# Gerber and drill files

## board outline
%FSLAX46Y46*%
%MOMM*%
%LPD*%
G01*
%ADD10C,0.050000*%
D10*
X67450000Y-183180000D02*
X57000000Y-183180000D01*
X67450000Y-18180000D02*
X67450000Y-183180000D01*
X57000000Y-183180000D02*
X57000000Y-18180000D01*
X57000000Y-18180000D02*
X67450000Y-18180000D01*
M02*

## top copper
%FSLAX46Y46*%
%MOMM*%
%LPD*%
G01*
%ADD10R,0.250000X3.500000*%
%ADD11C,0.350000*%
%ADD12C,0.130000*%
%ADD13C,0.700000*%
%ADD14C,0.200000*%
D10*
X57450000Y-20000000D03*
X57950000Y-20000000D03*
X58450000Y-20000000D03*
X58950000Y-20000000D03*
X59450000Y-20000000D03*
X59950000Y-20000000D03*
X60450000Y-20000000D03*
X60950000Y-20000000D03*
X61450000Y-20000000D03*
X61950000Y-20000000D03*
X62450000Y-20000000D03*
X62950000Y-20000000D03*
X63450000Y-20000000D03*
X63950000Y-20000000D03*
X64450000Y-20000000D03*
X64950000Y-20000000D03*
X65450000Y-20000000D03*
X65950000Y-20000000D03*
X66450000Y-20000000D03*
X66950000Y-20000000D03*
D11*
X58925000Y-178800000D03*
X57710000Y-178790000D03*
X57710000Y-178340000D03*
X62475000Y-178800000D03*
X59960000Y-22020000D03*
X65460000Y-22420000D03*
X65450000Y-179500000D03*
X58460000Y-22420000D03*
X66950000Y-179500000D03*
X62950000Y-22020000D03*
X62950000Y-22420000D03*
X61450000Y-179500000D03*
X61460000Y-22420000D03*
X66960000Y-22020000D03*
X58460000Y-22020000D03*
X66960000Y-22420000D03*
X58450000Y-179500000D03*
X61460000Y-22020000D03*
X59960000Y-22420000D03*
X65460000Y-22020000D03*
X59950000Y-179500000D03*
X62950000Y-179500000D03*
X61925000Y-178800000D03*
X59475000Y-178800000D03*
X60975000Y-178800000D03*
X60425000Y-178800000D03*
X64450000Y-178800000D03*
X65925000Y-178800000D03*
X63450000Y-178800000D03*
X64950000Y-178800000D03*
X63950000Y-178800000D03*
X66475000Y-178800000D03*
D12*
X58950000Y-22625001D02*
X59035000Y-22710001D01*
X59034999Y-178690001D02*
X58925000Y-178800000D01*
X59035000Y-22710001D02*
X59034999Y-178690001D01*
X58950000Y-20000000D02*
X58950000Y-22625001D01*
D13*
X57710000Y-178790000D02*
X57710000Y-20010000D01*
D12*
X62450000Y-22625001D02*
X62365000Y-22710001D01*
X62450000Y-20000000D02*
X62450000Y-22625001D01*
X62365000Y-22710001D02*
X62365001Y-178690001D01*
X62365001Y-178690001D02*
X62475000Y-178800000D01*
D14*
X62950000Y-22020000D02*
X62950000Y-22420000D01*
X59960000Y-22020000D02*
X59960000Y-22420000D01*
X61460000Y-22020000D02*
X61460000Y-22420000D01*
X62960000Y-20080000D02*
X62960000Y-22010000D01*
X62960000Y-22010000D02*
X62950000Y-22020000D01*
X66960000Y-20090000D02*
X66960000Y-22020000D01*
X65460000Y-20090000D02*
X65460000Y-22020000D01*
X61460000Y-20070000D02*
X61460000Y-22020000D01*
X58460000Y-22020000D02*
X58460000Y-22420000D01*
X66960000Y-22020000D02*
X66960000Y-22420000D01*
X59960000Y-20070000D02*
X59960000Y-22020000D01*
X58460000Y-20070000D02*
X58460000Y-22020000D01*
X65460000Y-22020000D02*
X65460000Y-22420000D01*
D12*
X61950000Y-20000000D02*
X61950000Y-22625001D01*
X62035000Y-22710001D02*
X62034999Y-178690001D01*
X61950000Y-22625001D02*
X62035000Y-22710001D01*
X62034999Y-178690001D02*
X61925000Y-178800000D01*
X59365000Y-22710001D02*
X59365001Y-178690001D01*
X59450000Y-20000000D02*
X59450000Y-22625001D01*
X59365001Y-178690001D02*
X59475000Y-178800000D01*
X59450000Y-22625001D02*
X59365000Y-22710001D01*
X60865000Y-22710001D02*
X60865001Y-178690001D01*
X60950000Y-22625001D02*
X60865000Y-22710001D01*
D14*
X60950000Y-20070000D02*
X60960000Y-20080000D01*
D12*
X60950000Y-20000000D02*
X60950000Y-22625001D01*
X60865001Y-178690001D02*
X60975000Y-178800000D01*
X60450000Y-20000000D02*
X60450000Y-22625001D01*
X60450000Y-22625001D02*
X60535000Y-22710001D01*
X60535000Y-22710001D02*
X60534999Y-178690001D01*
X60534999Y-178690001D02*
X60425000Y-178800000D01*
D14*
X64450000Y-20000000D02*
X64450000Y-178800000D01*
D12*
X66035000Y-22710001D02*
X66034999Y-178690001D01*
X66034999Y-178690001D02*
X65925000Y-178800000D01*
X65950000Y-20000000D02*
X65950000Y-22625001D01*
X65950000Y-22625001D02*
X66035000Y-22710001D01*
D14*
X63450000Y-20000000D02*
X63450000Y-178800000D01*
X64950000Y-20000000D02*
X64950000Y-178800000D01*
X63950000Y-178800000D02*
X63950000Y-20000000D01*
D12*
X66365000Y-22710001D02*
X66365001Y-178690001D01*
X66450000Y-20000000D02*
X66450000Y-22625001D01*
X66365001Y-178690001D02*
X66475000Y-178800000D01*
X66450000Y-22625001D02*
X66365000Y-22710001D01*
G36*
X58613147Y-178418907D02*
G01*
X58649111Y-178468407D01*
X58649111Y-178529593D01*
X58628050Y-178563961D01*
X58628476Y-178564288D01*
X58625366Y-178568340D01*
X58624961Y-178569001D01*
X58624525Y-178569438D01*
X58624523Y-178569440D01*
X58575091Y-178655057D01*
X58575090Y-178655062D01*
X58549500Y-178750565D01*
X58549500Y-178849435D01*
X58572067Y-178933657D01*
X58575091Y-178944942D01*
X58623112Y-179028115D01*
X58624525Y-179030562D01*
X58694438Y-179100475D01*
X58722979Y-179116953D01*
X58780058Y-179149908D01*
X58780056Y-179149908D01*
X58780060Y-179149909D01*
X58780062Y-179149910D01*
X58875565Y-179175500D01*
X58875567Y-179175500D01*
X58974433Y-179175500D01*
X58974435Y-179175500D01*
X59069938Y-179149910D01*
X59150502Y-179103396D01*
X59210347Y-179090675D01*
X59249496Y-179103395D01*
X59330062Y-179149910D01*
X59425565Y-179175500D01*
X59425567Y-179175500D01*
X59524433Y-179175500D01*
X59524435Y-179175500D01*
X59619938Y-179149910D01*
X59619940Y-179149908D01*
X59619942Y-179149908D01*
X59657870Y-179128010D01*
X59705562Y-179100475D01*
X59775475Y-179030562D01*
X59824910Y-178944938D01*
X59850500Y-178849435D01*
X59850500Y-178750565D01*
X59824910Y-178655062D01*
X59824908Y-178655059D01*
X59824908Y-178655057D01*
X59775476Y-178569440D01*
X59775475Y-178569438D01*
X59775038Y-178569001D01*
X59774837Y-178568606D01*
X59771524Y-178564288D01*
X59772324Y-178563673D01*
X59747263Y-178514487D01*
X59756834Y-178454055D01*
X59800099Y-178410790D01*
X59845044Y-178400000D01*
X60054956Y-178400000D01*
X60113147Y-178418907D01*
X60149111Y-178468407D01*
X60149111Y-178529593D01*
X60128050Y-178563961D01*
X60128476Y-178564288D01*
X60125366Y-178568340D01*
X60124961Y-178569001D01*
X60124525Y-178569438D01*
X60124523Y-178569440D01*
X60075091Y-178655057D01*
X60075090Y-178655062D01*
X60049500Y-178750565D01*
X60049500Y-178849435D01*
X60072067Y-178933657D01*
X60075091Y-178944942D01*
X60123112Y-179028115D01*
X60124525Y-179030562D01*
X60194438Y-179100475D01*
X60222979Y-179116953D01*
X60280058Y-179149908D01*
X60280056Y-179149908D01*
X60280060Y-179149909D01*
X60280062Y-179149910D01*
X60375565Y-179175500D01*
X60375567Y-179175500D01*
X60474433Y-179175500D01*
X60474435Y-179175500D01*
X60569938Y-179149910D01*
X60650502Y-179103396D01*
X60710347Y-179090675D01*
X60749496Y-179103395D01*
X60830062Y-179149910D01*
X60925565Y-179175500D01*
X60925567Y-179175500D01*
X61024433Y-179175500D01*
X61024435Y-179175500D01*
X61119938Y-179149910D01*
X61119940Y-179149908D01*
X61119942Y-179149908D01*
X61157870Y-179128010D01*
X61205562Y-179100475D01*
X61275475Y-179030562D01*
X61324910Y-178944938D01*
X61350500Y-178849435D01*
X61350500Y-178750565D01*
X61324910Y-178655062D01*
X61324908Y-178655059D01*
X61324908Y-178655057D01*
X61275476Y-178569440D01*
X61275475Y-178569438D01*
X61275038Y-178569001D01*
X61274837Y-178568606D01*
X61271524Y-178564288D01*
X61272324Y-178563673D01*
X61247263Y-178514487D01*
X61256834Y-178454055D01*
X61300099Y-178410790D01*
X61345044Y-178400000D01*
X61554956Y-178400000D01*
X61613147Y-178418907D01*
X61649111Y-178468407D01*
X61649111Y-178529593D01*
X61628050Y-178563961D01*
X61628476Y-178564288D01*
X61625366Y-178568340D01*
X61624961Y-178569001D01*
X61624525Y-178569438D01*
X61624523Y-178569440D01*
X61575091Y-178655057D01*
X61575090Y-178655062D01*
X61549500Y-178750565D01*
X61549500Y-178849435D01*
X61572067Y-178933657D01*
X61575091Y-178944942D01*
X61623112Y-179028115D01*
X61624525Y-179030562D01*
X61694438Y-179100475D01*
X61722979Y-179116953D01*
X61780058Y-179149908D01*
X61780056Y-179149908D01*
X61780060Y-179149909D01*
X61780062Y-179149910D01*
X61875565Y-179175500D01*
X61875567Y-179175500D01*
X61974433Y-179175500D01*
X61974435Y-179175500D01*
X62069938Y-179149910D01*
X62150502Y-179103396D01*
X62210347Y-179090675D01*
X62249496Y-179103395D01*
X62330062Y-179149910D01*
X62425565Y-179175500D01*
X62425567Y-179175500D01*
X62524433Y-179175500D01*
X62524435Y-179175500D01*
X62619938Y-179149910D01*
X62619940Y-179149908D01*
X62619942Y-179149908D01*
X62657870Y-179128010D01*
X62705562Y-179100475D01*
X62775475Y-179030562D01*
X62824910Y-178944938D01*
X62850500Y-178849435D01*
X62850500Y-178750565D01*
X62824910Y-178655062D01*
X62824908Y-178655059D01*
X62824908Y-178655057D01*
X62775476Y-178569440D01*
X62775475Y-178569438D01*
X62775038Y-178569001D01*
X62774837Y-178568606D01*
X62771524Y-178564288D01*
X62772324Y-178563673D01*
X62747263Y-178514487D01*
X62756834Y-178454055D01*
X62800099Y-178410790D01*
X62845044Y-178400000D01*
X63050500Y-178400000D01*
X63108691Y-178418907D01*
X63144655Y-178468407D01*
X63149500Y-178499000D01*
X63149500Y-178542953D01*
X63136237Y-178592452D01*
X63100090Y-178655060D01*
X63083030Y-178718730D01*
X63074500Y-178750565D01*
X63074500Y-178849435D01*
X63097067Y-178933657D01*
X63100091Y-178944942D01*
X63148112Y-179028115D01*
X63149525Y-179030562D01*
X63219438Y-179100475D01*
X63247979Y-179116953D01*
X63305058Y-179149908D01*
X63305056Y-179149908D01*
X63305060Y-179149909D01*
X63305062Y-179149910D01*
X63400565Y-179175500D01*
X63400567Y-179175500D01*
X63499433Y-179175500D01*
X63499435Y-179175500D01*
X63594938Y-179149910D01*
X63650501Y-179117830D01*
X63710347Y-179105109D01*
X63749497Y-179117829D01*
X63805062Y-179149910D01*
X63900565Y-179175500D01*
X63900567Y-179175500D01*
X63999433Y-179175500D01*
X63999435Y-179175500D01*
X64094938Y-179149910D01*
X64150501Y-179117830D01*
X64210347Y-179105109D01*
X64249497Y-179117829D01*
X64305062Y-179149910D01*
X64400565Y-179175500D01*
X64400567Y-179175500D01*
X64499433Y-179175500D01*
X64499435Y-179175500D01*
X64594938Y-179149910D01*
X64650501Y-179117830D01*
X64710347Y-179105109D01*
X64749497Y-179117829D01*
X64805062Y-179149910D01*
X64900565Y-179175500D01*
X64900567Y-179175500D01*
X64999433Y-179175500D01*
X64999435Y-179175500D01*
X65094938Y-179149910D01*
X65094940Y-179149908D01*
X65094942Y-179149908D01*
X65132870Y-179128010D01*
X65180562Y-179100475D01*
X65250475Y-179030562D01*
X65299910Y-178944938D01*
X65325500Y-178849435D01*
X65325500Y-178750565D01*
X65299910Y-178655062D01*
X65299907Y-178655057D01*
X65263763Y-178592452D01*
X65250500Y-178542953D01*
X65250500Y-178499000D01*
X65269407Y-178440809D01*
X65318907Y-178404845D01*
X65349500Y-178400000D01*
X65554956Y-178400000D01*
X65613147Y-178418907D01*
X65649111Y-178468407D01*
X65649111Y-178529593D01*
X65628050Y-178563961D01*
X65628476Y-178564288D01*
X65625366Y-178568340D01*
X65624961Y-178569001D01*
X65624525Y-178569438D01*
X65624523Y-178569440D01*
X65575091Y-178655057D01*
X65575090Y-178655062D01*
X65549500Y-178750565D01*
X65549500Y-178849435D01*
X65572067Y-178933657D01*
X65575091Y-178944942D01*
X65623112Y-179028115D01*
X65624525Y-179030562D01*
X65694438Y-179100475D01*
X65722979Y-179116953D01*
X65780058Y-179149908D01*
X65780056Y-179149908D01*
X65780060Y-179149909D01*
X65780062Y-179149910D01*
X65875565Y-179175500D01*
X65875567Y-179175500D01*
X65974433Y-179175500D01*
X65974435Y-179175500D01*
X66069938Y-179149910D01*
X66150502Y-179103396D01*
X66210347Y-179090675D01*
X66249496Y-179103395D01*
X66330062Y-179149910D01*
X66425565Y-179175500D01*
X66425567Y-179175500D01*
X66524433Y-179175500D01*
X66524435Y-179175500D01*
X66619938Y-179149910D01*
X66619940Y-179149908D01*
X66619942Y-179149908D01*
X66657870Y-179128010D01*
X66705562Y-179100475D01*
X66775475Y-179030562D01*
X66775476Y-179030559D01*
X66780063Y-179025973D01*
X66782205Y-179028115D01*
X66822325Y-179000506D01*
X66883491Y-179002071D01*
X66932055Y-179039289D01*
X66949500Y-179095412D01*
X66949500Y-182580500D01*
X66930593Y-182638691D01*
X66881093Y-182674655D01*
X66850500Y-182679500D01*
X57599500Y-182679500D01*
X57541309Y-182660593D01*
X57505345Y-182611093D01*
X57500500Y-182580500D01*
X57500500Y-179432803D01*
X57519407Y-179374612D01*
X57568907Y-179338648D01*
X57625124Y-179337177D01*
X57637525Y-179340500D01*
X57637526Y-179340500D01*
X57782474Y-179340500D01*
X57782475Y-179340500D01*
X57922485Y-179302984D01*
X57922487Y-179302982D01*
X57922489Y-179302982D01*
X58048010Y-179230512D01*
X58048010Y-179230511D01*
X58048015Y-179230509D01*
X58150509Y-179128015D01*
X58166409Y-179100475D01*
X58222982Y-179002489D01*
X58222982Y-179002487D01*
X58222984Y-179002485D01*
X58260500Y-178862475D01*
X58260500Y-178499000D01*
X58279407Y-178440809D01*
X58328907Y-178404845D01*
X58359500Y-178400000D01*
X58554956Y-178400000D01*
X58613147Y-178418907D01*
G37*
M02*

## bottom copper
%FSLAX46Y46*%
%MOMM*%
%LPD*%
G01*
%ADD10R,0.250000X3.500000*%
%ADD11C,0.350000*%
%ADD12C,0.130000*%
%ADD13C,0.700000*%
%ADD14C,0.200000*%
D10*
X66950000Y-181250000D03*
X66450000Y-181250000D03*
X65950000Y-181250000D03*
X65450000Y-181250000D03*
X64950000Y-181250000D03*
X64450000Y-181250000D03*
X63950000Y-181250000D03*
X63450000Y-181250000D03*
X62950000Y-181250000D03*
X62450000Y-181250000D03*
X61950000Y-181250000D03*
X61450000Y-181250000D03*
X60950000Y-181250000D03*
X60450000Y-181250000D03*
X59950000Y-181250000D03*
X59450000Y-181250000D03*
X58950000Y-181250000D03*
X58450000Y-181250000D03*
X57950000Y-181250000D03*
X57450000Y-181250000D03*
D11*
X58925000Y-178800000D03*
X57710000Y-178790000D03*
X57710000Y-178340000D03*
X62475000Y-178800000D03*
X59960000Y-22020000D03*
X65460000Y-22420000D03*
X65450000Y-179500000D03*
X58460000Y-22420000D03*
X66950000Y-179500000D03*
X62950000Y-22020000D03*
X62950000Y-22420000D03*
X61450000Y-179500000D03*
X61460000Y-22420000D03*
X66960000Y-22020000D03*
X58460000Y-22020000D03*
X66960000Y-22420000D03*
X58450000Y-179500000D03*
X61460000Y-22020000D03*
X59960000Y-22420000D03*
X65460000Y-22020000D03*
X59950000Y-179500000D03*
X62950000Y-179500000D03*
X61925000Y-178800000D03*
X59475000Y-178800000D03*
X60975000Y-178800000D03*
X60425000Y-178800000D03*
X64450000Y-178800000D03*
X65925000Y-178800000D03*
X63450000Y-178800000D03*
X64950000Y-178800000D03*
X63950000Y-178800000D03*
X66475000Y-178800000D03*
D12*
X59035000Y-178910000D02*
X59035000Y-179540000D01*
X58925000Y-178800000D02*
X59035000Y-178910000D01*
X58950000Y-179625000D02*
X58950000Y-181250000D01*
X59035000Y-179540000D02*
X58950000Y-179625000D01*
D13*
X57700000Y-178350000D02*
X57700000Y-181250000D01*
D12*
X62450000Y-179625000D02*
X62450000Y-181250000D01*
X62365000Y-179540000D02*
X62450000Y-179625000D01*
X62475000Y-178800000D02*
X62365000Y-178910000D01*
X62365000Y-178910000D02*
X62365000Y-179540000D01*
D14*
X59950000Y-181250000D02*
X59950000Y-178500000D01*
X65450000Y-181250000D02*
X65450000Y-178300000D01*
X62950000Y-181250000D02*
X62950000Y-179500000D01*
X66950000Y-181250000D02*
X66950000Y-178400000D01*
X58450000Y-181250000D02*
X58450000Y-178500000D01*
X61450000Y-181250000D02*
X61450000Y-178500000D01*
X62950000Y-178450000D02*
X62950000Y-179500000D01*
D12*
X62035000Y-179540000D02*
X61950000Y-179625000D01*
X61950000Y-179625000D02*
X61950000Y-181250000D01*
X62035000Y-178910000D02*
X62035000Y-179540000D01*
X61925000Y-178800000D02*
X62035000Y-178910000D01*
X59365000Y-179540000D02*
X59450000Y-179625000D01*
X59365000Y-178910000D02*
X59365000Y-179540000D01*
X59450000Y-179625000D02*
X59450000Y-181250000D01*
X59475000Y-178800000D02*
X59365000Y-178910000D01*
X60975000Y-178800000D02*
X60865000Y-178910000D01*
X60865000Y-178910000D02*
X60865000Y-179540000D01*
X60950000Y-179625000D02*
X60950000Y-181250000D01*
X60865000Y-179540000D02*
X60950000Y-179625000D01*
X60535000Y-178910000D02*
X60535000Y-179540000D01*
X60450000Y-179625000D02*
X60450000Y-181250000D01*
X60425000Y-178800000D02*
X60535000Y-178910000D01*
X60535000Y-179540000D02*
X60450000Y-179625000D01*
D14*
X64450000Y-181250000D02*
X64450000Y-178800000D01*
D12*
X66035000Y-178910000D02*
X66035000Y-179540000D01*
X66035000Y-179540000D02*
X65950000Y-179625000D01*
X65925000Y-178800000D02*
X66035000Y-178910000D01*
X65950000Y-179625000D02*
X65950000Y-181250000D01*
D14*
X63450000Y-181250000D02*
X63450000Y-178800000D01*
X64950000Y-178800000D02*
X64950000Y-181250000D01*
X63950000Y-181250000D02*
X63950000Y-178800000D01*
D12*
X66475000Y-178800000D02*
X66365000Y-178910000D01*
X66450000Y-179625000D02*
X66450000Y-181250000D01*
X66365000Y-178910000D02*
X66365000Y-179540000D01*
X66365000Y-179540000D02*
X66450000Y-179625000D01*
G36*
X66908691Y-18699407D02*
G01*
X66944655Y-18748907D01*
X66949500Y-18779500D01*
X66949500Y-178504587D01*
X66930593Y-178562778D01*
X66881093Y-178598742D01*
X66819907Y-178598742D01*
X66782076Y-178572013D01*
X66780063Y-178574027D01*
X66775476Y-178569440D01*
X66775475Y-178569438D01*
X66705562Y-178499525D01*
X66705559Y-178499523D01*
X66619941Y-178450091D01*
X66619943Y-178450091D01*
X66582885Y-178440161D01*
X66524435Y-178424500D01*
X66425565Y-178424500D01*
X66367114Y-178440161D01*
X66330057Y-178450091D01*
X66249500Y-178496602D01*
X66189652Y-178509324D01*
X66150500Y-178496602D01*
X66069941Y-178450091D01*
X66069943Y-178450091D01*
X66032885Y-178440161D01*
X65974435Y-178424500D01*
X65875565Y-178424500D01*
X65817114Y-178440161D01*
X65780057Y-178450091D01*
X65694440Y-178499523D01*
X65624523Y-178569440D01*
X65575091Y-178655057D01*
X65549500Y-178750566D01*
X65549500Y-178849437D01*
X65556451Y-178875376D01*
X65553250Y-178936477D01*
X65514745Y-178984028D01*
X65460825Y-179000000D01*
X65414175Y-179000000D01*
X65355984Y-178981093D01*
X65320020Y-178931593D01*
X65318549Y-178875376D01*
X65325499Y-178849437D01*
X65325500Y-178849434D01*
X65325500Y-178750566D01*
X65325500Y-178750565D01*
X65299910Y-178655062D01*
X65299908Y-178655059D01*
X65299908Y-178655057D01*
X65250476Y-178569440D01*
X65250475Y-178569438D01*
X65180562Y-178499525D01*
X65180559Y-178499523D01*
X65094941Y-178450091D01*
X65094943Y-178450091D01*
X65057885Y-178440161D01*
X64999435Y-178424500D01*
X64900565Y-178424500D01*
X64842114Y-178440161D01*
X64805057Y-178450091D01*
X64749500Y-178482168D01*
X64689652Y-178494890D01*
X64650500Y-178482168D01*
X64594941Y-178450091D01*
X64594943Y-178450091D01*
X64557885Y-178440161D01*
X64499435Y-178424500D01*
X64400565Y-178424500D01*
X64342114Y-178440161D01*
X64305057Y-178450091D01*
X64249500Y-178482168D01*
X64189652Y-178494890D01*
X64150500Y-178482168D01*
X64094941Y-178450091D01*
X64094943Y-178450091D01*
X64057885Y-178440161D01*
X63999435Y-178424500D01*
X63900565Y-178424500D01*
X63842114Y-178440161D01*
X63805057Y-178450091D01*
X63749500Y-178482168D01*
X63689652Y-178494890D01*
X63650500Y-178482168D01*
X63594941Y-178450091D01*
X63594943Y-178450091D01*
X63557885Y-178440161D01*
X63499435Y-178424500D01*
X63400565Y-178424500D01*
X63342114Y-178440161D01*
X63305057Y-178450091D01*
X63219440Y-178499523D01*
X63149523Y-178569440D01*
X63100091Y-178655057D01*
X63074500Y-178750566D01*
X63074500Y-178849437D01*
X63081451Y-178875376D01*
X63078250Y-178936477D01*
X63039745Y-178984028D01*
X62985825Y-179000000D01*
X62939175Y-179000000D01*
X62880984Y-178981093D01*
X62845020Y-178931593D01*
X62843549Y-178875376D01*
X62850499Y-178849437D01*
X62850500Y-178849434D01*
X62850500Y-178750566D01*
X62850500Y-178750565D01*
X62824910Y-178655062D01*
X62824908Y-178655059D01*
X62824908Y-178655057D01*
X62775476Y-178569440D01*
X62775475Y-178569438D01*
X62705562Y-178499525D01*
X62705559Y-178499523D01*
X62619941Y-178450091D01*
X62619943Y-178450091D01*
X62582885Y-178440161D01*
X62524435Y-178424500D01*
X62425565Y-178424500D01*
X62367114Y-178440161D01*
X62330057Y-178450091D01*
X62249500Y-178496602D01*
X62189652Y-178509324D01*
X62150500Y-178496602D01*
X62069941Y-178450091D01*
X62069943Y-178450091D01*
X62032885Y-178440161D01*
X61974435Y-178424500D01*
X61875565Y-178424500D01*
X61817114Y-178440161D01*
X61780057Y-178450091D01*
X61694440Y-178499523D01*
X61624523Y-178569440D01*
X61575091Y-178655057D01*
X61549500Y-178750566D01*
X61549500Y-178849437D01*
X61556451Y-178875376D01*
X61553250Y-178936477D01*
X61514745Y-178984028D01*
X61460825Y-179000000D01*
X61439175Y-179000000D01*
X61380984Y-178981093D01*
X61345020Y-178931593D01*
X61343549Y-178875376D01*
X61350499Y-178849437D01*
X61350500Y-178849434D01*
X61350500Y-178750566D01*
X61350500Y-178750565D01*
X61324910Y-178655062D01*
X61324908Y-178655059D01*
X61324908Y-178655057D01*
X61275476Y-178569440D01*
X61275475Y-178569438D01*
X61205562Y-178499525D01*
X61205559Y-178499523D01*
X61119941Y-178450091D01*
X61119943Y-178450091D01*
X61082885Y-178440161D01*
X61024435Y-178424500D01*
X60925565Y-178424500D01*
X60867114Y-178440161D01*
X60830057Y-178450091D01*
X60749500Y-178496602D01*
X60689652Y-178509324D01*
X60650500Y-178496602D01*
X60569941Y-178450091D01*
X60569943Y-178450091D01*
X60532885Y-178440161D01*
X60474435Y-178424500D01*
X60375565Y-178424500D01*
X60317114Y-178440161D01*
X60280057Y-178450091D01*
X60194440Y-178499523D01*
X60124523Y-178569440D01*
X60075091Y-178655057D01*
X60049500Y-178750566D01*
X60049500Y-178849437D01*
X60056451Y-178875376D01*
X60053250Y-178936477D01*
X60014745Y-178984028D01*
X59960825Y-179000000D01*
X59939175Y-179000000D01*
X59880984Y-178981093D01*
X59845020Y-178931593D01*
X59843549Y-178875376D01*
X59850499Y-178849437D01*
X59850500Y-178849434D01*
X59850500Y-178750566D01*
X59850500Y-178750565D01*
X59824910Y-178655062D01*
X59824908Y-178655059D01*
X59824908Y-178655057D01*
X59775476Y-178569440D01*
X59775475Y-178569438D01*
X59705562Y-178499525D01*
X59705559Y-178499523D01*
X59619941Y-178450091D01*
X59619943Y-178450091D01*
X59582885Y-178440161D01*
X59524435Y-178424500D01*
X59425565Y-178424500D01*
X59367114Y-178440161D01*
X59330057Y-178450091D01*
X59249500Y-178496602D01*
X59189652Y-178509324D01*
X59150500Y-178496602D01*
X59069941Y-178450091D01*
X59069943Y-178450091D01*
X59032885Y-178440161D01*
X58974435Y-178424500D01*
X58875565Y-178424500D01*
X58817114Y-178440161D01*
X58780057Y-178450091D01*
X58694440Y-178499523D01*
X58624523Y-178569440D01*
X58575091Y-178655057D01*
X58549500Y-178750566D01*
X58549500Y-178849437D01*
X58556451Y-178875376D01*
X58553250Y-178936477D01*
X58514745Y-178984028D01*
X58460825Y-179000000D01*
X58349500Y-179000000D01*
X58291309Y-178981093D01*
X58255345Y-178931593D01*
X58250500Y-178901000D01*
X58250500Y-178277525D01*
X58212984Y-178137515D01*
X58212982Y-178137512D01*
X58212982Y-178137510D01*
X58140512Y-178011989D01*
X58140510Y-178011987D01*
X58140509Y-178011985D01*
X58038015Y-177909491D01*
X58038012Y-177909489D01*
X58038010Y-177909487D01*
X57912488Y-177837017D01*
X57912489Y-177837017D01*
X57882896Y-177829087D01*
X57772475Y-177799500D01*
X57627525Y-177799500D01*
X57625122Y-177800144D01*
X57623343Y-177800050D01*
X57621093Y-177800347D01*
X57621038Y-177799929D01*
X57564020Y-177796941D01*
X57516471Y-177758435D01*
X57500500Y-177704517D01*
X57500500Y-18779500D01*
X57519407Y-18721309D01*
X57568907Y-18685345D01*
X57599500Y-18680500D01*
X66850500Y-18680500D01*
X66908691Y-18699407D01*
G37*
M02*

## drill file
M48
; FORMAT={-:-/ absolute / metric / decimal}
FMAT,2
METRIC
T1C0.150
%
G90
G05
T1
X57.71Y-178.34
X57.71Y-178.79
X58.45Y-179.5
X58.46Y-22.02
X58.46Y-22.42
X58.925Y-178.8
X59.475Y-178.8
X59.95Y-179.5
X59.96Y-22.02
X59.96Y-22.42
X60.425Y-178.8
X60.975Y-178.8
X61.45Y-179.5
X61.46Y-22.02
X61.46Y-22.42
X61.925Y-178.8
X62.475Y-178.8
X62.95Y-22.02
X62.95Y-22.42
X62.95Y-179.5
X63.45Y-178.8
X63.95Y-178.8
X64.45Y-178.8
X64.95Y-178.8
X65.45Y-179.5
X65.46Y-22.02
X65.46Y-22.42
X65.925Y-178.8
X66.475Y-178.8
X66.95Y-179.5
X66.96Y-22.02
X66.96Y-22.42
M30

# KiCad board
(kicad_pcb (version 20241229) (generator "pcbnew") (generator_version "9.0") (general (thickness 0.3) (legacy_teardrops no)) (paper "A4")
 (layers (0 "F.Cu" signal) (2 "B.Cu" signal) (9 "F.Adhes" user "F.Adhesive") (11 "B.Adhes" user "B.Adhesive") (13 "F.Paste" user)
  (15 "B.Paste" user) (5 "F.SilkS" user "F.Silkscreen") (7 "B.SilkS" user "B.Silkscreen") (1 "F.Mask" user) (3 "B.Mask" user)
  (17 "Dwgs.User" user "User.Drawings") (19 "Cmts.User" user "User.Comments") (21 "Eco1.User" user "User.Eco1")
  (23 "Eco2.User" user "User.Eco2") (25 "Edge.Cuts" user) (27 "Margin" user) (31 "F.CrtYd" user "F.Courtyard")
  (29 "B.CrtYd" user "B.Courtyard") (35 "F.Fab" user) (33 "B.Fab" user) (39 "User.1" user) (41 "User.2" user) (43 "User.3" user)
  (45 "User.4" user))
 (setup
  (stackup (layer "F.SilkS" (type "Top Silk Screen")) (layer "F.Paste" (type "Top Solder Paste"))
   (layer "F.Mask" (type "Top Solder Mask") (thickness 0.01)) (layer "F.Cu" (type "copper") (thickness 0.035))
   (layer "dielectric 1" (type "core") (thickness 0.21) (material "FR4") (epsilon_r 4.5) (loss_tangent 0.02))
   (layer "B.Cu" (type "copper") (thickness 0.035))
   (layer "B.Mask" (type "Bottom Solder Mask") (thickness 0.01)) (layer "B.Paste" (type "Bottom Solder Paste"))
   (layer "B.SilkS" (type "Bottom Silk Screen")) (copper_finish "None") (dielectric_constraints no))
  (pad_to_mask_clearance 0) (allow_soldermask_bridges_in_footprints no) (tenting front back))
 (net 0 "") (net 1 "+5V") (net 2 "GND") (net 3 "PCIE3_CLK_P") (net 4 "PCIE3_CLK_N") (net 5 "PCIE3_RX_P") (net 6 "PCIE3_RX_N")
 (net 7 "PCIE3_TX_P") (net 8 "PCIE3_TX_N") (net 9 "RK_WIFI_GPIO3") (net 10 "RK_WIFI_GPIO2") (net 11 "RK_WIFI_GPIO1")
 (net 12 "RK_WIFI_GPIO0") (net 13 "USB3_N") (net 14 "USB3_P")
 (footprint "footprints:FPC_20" (layer "F.Cu") (at 62.2 20 180)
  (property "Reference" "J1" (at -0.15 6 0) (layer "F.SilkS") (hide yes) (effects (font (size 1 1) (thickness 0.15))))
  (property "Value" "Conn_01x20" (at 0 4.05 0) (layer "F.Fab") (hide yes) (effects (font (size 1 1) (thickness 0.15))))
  (pad "1" smd rect (at 4.75 0 180) (size 0.25 3.5) (layers "F.Cu" "F.Mask" "F.Paste") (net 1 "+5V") (thermal_bridge_angle 45))
  (pad "2" smd rect (at 4.25 0 180) (size 0.25 3.5) (layers "F.Cu" "F.Mask" "F.Paste") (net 1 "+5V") (thermal_bridge_angle 45))
  (pad "3" smd rect (at 3.75 0 180) (size 0.25 3.5) (layers "F.Cu" "F.Mask" "F.Paste") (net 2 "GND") (thermal_bridge_angle 45))
  (pad "4" smd rect (at 3.25 0 180) (size 0.25 3.5) (layers "F.Cu" "F.Mask" "F.Paste") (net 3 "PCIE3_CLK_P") (thermal_bridge_angle 45))
  (pad "5" smd rect (at 2.75 0 180) (size 0.25 3.5) (layers "F.Cu" "F.Mask" "F.Paste") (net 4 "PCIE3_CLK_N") (thermal_bridge_angle 45))
  (pad "6" smd rect (at 2.25 0 180) (size 0.25 3.5) (layers "F.Cu" "F.Mask" "F.Paste") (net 2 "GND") (thermal_bridge_angle 45))
  (pad "7" smd rect (at 1.75 0 180) (size 0.25 3.5) (layers "F.Cu" "F.Mask" "F.Paste") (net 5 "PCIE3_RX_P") (thermal_bridge_angle 45))
  (pad "8" smd rect (at 1.25 0 180) (size 0.25 3.5) (layers "F.Cu" "F.Mask" "F.Paste") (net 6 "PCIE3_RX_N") (thermal_bridge_angle 45))
  (pad "9" smd rect (at 0.75 0 180) (size 0.25 3.5) (layers "F.Cu" "F.Mask" "F.Paste") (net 2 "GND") (thermal_bridge_angle 45))
  (pad "10" smd rect (at 0.25 0 180) (size 0.25 3.5) (layers "F.Cu" "F.Mask" "F.Paste") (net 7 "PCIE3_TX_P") (thermal_bridge_angle 45))
  (pad "11" smd rect (at -0.25 0 180) (size 0.25 3.5) (layers "F.Cu" "F.Mask" "F.Paste") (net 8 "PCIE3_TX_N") (thermal_bridge_angle 45))
  (pad "12" smd rect (at -0.75 0 180) (size 0.25 3.5) (layers "F.Cu" "F.Mask" "F.Paste") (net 2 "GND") (thermal_bridge_angle 45))
  (pad "13" smd rect (at -1.25 0 180) (size 0.25 3.5) (layers "F.Cu" "F.Mask" "F.Paste") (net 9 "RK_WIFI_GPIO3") (thermal_bridge_angle 45))
  (pad "14" smd rect (at -1.75 0 180) (size 0.25 3.5) (layers "F.Cu" "F.Mask" "F.Paste") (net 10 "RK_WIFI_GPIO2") (thermal_bridge_angle 45))
  (pad "15" smd rect (at -2.25 0 180) (size 0.25 3.5) (layers "F.Cu" "F.Mask" "F.Paste") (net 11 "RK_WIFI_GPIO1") (thermal_bridge_angle 45))
  (pad "16" smd rect (at -2.75 0 180) (size 0.25 3.5) (layers "F.Cu" "F.Mask" "F.Paste") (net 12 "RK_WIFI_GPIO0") (thermal_bridge_angle 45))
  (pad "17" smd rect (at -3.25 0 180) (size 0.25 3.5) (layers "F.Cu" "F.Mask" "F.Paste") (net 2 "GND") (thermal_bridge_angle 45))
  (pad "18" smd rect (at -3.75 0 180) (size 0.25 3.5) (layers "F.Cu" "F.Mask" "F.Paste") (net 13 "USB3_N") (thermal_bridge_angle 45))
  (pad "19" smd rect (at -4.25 0 180) (size 0.25 3.5) (layers "F.Cu" "F.Mask" "F.Paste") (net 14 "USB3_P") (thermal_bridge_angle 45))
  (pad "20" smd rect (at -4.75 0 180) (size 0.25 3.5) (layers "F.Cu" "F.Mask" "F.Paste") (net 2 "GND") (thermal_bridge_angle 45)))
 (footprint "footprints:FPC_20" (layer "B.Cu") (at 62.2 181.25)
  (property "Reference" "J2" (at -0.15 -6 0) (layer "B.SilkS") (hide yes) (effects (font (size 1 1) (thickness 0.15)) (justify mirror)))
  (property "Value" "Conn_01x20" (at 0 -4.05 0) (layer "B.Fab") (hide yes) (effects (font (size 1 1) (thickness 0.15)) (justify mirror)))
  (pad "1" smd rect (at 4.75 0) (size 0.25 3.5) (layers "B.Cu" "B.Mask" "B.Paste") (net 2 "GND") (thermal_bridge_angle 45))
  (pad "2" smd rect (at 4.25 0) (size 0.25 3.5) (layers "B.Cu" "B.Mask" "B.Paste") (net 14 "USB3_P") (thermal_bridge_angle 45))
  (pad "3" smd rect (at 3.75 0) (size 0.25 3.5) (layers "B.Cu" "B.Mask" "B.Paste") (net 13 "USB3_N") (thermal_bridge_angle 45))
  (pad "4" smd rect (at 3.25 0) (size 0.25 3.5) (layers "B.Cu" "B.Mask" "B.Paste") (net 2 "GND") (thermal_bridge_angle 45))
  (pad "5" smd rect (at 2.75 0) (size 0.25 3.5) (layers "B.Cu" "B.Mask" "B.Paste") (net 12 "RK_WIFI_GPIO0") (thermal_bridge_angle 45))
  (pad "6" smd rect (at 2.25 0) (size 0.25 3.5) (layers "B.Cu" "B.Mask" "B.Paste") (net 11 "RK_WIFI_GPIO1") (thermal_bridge_angle 45))
  (pad "7" smd rect (at 1.75 0) (size 0.25 3.5) (layers "B.Cu" "B.Mask" "B.Paste") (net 10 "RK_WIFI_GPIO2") (thermal_bridge_angle 45))
  (pad "8" smd rect (at 1.25 0) (size 0.25 3.5) (layers "B.Cu" "B.Mask" "B.Paste") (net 9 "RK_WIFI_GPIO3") (thermal_bridge_angle 45))
  (pad "9" smd rect (at 0.75 0) (size 0.25 3.5) (layers "B.Cu" "B.Mask" "B.Paste") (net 2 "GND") (thermal_bridge_angle 45))
  (pad "10" smd rect (at 0.25 0) (size 0.25 3.5) (layers "B.Cu" "B.Mask" "B.Paste") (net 8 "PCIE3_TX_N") (thermal_bridge_angle 45))
  (pad "11" smd rect (at -0.25 0) (size 0.25 3.5) (layers "B.Cu" "B.Mask" "B.Paste") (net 7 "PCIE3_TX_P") (thermal_bridge_angle 45))
  (pad "12" smd rect (at -0.75 0) (size 0.25 3.5) (layers "B.Cu" "B.Mask" "B.Paste") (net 2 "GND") (thermal_bridge_angle 45))
  (pad "13" smd rect (at -1.25 0) (size 0.25 3.5) (layers "B.Cu" "B.Mask" "B.Paste") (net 6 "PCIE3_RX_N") (thermal_bridge_angle 45))
  (pad "14" smd rect (at -1.75 0) (size 0.25 3.5) (layers "B.Cu" "B.Mask" "B.Paste") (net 5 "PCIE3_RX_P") (thermal_bridge_angle 45))
  (pad "15" smd rect (at -2.25 0) (size 0.25 3.5) (layers "B.Cu" "B.Mask" "B.Paste") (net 2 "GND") (thermal_bridge_angle 45))
  (pad "16" smd rect (at -2.75 0) (size 0.25 3.5) (layers "B.Cu" "B.Mask" "B.Paste") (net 4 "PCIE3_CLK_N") (thermal_bridge_angle 45))
  (pad "17" smd rect (at -3.25 0) (size 0.25 3.5) (layers "B.Cu" "B.Mask" "B.Paste") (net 3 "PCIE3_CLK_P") (thermal_bridge_angle 45))
  (pad "18" smd rect (at -3.75 0) (size 0.25 3.5) (layers "B.Cu" "B.Mask" "B.Paste") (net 2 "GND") (thermal_bridge_angle 45))
  (pad "19" smd rect (at -4.25 0) (size 0.25 3.5) (layers "B.Cu" "B.Mask" "B.Paste") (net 1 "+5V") (thermal_bridge_angle 45))
  (pad "20" smd rect (at -4.75 0) (size 0.25 3.5) (layers "B.Cu" "B.Mask" "B.Paste") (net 1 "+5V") (thermal_bridge_angle 45)))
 (gr_line (start 67.45 183.18) (end 57 183.18) (stroke (width 0.05) (type solid)) (layer "Edge.Cuts"))
 (gr_line (start 67.45 18.18) (end 67.45 183.18) (stroke (width 0.05) (type solid)) (layer "Edge.Cuts"))
 (gr_line (start 57 183.18) (end 57 18.18) (stroke (width 0.05) (type solid)) (layer "Edge.Cuts"))
 (gr_line (start 57 18.18) (end 67.45 18.18) (stroke (width 0.05) (type solid)) (layer "Edge.Cuts"))
 (segment (start 58.95 22.625001) (end 59.035 22.710001) (width 0.13) (layer "F.Cu") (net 3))
 (segment (start 59.034999 178.690001) (end 58.925 178.8) (width 0.13) (layer "F.Cu") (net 3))
 (segment (start 59.035 22.710001) (end 59.034999 178.690001) (width 0.13) (layer "F.Cu") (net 3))
 (segment (start 58.95 20) (end 58.95 22.625001) (width 0.13) (layer "F.Cu") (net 3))
 (via (at 58.925 178.8) (size 0.35) (drill 0.15) (layers "F.Cu" "B.Cu") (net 3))
 (segment (start 59.035 178.91) (end 59.035 179.54) (width 0.13) (layer "B.Cu") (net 3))
 (segment (start 58.925 178.8) (end 59.035 178.91) (width 0.13) (layer "B.Cu") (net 3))
 (segment (start 58.95 179.625) (end 58.95 181.25) (width 0.13) (layer "B.Cu") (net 3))
 (segment (start 59.035 179.54) (end 58.95 179.625) (width 0.13) (layer "B.Cu") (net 3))
 (segment (start 57.71 178.79) (end 57.71 20.01) (width 0.7) (layer "F.Cu") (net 1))
 (via (at 57.71 178.79) (size 0.35) (drill 0.15) (layers "F.Cu" "B.Cu") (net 1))
 (via (at 57.71 178.34) (size 0.35) (drill 0.15) (layers "F.Cu" "B.Cu") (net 1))
 (segment (start 57.7 178.35) (end 57.7 181.25) (width 0.7) (layer "B.Cu") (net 1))
 (segment (start 62.45 22.625001) (end 62.365 22.710001) (width 0.13) (layer "F.Cu") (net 8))
 (segment (start 62.45 20) (end 62.45 22.625001) (width 0.13) (layer "F.Cu") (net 8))
 (segment (start 62.365 22.710001) (end 62.365001 178.690001) (width 0.13) (layer "F.Cu") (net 8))
 (segment (start 62.365001 178.690001) (end 62.475 178.8) (width 0.13) (layer "F.Cu") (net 8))
 (via (at 62.475 178.8) (size 0.35) (drill 0.15) (layers "F.Cu" "B.Cu") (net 8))
 (segment (start 62.45 179.625) (end 62.45 181.25) (width 0.13) (layer "B.Cu") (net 8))
 (segment (start 62.365 179.54) (end 62.45 179.625) (width 0.13) (layer "B.Cu") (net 8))
 (segment (start 62.475 178.8) (end 62.365 178.91) (width 0.13) (layer "B.Cu") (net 8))
 (segment (start 62.365 178.91) (end 62.365 179.54) (width 0.13) (layer "B.Cu") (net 8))
 (segment (start 62.95 22.02) (end 62.95 22.42) (width 0.2) (layer "F.Cu") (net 2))
 (segment (start 59.96 22.02) (end 59.96 22.42) (width 0.2) (layer "F.Cu") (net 2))
 (segment (start 61.46 22.02) (end 61.46 22.42) (width 0.2) (layer "F.Cu") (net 2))
 (segment (start 62.96 20.08) (end 62.96 22.01) (width 0.2) (layer "F.Cu") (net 2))
 (segment (start 62.96 22.01) (end 62.95 22.02) (width 0.2) (layer "F.Cu") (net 2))
 (segment (start 66.96 20.09) (end 66.96 22.02) (width 0.2) (layer "F.Cu") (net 2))
 (segment (start 65.46 20.09) (end 65.46 22.02) (width 0.2) (layer "F.Cu") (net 2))
 (segment (start 61.46 20.07) (end 61.46 22.02) (width 0.2) (layer "F.Cu") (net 2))
 (segment (start 58.46 22.02) (end 58.46 22.42) (width 0.2) (layer "F.Cu") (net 2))
 (segment (start 66.96 22.02) (end 66.96 22.42) (width 0.2) (layer "F.Cu") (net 2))
 (segment (start 59.96 20.07) (end 59.96 22.02) (width 0.2) (layer "F.Cu") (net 2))
 (segment (start 58.46 20.07) (end 58.46 22.02) (width 0.2) (layer "F.Cu") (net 2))
 (segment (start 65.46 22.02) (end 65.46 22.42) (width 0.2) (layer "F.Cu") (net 2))
 (via (at 59.96 22.02) (size 0.35) (drill 0.15) (layers "F.Cu" "B.Cu") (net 2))
 (via (at 65.46 22.42) (size 0.35) (drill 0.15) (layers "F.Cu" "B.Cu") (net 2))
 (via (at 65.45 179.5) (size 0.35) (drill 0.15) (layers "F.Cu" "B.Cu") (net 2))
 (via (at 58.46 22.42) (size 0.35) (drill 0.15) (layers "F.Cu" "B.Cu") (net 2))
 (via (at 66.95 179.5) (size 0.35) (drill 0.15) (layers "F.Cu" "B.Cu") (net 2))
 (via (at 62.95 22.02) (size 0.35) (drill 0.15) (layers "F.Cu" "B.Cu") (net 2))
 (via (at 62.95 22.42) (size 0.35) (drill 0.15) (layers "F.Cu" "B.Cu") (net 2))
 (via (at 61.45 179.5) (size 0.35) (drill 0.15) (layers "F.Cu" "B.Cu") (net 2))
 (via (at 61.46 22.42) (size 0.35) (drill 0.15) (layers "F.Cu" "B.Cu") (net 2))
 (via (at 66.96 22.02) (size 0.35) (drill 0.15) (layers "F.Cu" "B.Cu") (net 2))
 (via (at 58.46 22.02) (size 0.35) (drill 0.15) (layers "F.Cu" "B.Cu") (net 2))
 (via (at 66.96 22.42) (size 0.35) (drill 0.15) (layers "F.Cu" "B.Cu") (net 2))
 (via (at 58.45 179.5) (size 0.35) (drill 0.15) (layers "F.Cu" "B.Cu") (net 2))
 (via (at 61.46 22.02) (size 0.35) (drill 0.15) (layers "F.Cu" "B.Cu") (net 2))
 (via (at 59.96 22.42) (size 0.35) (drill 0.15) (layers "F.Cu" "B.Cu") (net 2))
 (via (at 65.46 22.02) (size 0.35) (drill 0.15) (layers "F.Cu" "B.Cu") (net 2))
 (via (at 59.95 179.5) (size 0.35) (drill 0.15) (layers "F.Cu" "B.Cu") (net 2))
 (via (at 62.95 179.5) (size 0.35) (drill 0.15) (layers "F.Cu" "B.Cu") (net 2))
 (segment (start 59.95 181.25) (end 59.95 178.5) (width 0.2) (layer "B.Cu") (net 2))
 (segment (start 65.45 181.25) (end 65.45 178.3) (width 0.2) (layer "B.Cu") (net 2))
 (segment (start 62.95 181.25) (end 62.95 179.5) (width 0.2) (layer "B.Cu") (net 2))
 (segment (start 66.95 181.25) (end 66.95 178.4) (width 0.2) (layer "B.Cu") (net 2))
 (segment (start 58.45 181.25) (end 58.45 178.5) (width 0.2) (layer "B.Cu") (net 2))
 (segment (start 61.45 181.25) (end 61.45 178.5) (width 0.2) (layer "B.Cu") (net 2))
 (segment (start 62.95 178.45) (end 62.95 179.5) (width 0.2) (layer "B.Cu") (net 2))
 (segment (start 61.95 20) (end 61.95 22.625001) (width 0.13) (layer "F.Cu") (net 7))
 (segment (start 62.035 22.710001) (end 62.034999 178.690001) (width 0.13) (layer "F.Cu") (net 7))
 (segment (start 61.95 22.625001) (end 62.035 22.710001) (width 0.13) (layer "F.Cu") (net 7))
 (segment (start 62.034999 178.690001) (end 61.925 178.8) (width 0.13) (layer "F.Cu") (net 7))
 (via (at 61.925 178.8) (size 0.35) (drill 0.15) (layers "F.Cu" "B.Cu") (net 7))
 (segment (start 62.035 179.54) (end 61.95 179.625) (width 0.13) (layer "B.Cu") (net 7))
 (segment (start 61.95 179.625) (end 61.95 181.25) (width 0.13) (layer "B.Cu") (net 7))
 (segment (start 62.035 178.91) (end 62.035 179.54) (width 0.13) (layer "B.Cu") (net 7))
 (segment (start 61.925 178.8) (end 62.035 178.91) (width 0.13) (layer "B.Cu") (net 7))
 (segment (start 59.365 22.710001) (end 59.365001 178.690001) (width 0.13) (layer "F.Cu") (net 4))
 (segment (start 59.45 20) (end 59.45 22.625001) (width 0.13) (layer "F.Cu") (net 4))
 (segment (start 59.365001 178.690001) (end 59.475 178.8) (width 0.13) (layer "F.Cu") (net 4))
 (segment (start 59.45 22.625001) (end 59.365 22.710001) (width 0.13) (layer "F.Cu") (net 4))
 (via (at 59.475 178.8) (size 0.35) (drill 0.15) (layers "F.Cu" "B.Cu") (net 4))
 (segment (start 59.365 179.54) (end 59.45 179.625) (width 0.13) (layer "B.Cu") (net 4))
 (segment (start 59.365 178.91) (end 59.365 179.54) (width 0.13) (layer "B.Cu") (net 4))
 (segment (start 59.45 179.625) (end 59.45 181.25) (width 0.13) (layer "B.Cu") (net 4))
 (segment (start 59.475 178.8) (end 59.365 178.91) (width 0.13) (layer "B.Cu") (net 4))
 (segment (start 60.865 22.710001) (end 60.865001 178.690001) (width 0.13) (layer "F.Cu") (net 6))
 (segment (start 60.95 22.625001) (end 60.865 22.710001) (width 0.13) (layer "F.Cu") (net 6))
 (segment (start 60.95 20.07) (end 60.96 20.08) (width 0.2) (layer "F.Cu") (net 6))
 (segment (start 60.95 20) (end 60.95 22.625001) (width 0.13) (layer "F.Cu") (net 6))
 (segment (start 60.865001 178.690001) (end 60.975 178.8) (width 0.13) (layer "F.Cu") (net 6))
 (via (at 60.975 178.8) (size 0.35) (drill 0.15) (layers "F.Cu" "B.Cu") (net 6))
 (segment (start 60.975 178.8) (end 60.865 178.91) (width 0.13) (layer "B.Cu") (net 6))
 (segment (start 60.865 178.91) (end 60.865 179.54) (width 0.13) (layer "B.Cu") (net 6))
 (segment (start 60.95 179.625) (end 60.95 181.25) (width 0.13) (layer "B.Cu") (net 6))
 (segment (start 60.865 179.54) (end 60.95 179.625) (width 0.13) (layer "B.Cu") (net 6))
 (segment (start 60.45 20) (end 60.45 22.625001) (width 0.13) (layer "F.Cu") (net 5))
 (segment (start 60.45 22.625001) (end 60.535 22.710001) (width 0.13) (layer "F.Cu") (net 5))
 (segment (start 60.535 22.710001) (end 60.534999 178.690001) (width 0.13) (layer "F.Cu") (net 5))
 (segment (start 60.534999 178.690001) (end 60.425 178.8) (width 0.13) (layer "F.Cu") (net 5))
 (via (at 60.425 178.8) (size 0.35) (drill 0.15) (layers "F.Cu" "B.Cu") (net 5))
 (segment (start 60.535 178.91) (end 60.535 179.54) (width 0.13) (layer "B.Cu") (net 5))
 (segment (start 60.45 179.625) (end 60.45 181.25) (width 0.13) (layer "B.Cu") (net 5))
 (segment (start 60.425 178.8) (end 60.535 178.91) (width 0.13) (layer "B.Cu") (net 5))
 (segment (start 60.535 179.54) (end 60.45 179.625) (width 0.13) (layer "B.Cu") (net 5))
 (segment (start 64.45 20) (end 64.45 178.8) (width 0.2) (layer "F.Cu") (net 11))
 (via (at 64.45 178.8) (size 0.35) (drill 0.15) (layers "F.Cu" "B.Cu") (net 11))
 (segment (start 64.45 181.25) (end 64.45 178.8) (width 0.2) (layer "B.Cu") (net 11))
 (segment (start 66.035 22.710001) (end 66.034999 178.690001) (width 0.13) (layer "F.Cu") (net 13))
 (segment (start 66.034999 178.690001) (end 65.925 178.8) (width 0.13) (layer "F.Cu") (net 13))
 (segment (start 65.95 20) (end 65.95 22.625001) (width 0.13) (layer "F.Cu") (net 13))
 (segment (start 65.95 22.625001) (end 66.035 22.710001) (width 0.13) (layer "F.Cu") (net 13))
 (via (at 65.925 178.8) (size 0.35) (drill 0.15) (layers "F.Cu" "B.Cu") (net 13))
 (segment (start 66.035 178.91) (end 66.035 179.54) (width 0.13) (layer "B.Cu") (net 13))
 (segment (start 66.035 179.54) (end 65.95 179.625) (width 0.13) (layer "B.Cu") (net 13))
 (segment (start 65.925 178.8) (end 66.035 178.91) (width 0.13) (layer "B.Cu") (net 13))
 (segment (start 65.95 179.625) (end 65.95 181.25) (width 0.13) (layer "B.Cu") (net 13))
 (segment (start 63.45 20) (end 63.45 178.8) (width 0.2) (layer "F.Cu") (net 9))
 (via (at 63.45 178.8) (size 0.35) (drill 0.15) (layers "F.Cu" "B.Cu") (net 9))
 (segment (start 63.45 181.25) (end 63.45 178.8) (width 0.2) (layer "B.Cu") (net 9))
 (segment (start 64.95 20) (end 64.95 178.8) (width 0.2) (layer "F.Cu") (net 12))
 (via (at 64.95 178.8) (size 0.35) (drill 0.15) (layers "F.Cu" "B.Cu") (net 12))
 (segment (start 64.95 178.8) (end 64.95 181.25) (width 0.2) (layer "B.Cu") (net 12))
 (segment (start 63.95 178.8) (end 63.95 20) (width 0.2) (layer "F.Cu") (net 10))
 (via (at 63.95 178.8) (size 0.35) (drill 0.15) (layers "F.Cu" "B.Cu") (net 10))
 (segment (start 63.95 181.25) (end 63.95 178.8) (width 0.2) (layer "B.Cu") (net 10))
 (segment (start 66.365 22.710001) (end 66.365001 178.690001) (width 0.13) (layer "F.Cu") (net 14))
 (segment (start 66.45 20) (end 66.45 22.625001) (width 0.13) (layer "F.Cu") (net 14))
 (segment (start 66.365001 178.690001) (end 66.475 178.8) (width 0.13) (layer "F.Cu") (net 14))
 (segment (start 66.45 22.625001) (end 66.365 22.710001) (width 0.13) (layer "F.Cu") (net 14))
 (via (at 66.475 178.8) (size 0.35) (drill 0.15) (layers "F.Cu" "B.Cu") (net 14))
 (segment (start 66.475 178.8) (end 66.365 178.91) (width 0.13) (layer "B.Cu") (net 14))
 (segment (start 66.45 179.625) (end 66.45 181.25) (width 0.13) (layer "B.Cu") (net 14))
 (segment (start 66.365 178.91) (end 66.365 179.54) (width 0.13) (layer "B.Cu") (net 14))
 (segment (start 66.365 179.54) (end 66.45 179.625) (width 0.13) (layer "B.Cu") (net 14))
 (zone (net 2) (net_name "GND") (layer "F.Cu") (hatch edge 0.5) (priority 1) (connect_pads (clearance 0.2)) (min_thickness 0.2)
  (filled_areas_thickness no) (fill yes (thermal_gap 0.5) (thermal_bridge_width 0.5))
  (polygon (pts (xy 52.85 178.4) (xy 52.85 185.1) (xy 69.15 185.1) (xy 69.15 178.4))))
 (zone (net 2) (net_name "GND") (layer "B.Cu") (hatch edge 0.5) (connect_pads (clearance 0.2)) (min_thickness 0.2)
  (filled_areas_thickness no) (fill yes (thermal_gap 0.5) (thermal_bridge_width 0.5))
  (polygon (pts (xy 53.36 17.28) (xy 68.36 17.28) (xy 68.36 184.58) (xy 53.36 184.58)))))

